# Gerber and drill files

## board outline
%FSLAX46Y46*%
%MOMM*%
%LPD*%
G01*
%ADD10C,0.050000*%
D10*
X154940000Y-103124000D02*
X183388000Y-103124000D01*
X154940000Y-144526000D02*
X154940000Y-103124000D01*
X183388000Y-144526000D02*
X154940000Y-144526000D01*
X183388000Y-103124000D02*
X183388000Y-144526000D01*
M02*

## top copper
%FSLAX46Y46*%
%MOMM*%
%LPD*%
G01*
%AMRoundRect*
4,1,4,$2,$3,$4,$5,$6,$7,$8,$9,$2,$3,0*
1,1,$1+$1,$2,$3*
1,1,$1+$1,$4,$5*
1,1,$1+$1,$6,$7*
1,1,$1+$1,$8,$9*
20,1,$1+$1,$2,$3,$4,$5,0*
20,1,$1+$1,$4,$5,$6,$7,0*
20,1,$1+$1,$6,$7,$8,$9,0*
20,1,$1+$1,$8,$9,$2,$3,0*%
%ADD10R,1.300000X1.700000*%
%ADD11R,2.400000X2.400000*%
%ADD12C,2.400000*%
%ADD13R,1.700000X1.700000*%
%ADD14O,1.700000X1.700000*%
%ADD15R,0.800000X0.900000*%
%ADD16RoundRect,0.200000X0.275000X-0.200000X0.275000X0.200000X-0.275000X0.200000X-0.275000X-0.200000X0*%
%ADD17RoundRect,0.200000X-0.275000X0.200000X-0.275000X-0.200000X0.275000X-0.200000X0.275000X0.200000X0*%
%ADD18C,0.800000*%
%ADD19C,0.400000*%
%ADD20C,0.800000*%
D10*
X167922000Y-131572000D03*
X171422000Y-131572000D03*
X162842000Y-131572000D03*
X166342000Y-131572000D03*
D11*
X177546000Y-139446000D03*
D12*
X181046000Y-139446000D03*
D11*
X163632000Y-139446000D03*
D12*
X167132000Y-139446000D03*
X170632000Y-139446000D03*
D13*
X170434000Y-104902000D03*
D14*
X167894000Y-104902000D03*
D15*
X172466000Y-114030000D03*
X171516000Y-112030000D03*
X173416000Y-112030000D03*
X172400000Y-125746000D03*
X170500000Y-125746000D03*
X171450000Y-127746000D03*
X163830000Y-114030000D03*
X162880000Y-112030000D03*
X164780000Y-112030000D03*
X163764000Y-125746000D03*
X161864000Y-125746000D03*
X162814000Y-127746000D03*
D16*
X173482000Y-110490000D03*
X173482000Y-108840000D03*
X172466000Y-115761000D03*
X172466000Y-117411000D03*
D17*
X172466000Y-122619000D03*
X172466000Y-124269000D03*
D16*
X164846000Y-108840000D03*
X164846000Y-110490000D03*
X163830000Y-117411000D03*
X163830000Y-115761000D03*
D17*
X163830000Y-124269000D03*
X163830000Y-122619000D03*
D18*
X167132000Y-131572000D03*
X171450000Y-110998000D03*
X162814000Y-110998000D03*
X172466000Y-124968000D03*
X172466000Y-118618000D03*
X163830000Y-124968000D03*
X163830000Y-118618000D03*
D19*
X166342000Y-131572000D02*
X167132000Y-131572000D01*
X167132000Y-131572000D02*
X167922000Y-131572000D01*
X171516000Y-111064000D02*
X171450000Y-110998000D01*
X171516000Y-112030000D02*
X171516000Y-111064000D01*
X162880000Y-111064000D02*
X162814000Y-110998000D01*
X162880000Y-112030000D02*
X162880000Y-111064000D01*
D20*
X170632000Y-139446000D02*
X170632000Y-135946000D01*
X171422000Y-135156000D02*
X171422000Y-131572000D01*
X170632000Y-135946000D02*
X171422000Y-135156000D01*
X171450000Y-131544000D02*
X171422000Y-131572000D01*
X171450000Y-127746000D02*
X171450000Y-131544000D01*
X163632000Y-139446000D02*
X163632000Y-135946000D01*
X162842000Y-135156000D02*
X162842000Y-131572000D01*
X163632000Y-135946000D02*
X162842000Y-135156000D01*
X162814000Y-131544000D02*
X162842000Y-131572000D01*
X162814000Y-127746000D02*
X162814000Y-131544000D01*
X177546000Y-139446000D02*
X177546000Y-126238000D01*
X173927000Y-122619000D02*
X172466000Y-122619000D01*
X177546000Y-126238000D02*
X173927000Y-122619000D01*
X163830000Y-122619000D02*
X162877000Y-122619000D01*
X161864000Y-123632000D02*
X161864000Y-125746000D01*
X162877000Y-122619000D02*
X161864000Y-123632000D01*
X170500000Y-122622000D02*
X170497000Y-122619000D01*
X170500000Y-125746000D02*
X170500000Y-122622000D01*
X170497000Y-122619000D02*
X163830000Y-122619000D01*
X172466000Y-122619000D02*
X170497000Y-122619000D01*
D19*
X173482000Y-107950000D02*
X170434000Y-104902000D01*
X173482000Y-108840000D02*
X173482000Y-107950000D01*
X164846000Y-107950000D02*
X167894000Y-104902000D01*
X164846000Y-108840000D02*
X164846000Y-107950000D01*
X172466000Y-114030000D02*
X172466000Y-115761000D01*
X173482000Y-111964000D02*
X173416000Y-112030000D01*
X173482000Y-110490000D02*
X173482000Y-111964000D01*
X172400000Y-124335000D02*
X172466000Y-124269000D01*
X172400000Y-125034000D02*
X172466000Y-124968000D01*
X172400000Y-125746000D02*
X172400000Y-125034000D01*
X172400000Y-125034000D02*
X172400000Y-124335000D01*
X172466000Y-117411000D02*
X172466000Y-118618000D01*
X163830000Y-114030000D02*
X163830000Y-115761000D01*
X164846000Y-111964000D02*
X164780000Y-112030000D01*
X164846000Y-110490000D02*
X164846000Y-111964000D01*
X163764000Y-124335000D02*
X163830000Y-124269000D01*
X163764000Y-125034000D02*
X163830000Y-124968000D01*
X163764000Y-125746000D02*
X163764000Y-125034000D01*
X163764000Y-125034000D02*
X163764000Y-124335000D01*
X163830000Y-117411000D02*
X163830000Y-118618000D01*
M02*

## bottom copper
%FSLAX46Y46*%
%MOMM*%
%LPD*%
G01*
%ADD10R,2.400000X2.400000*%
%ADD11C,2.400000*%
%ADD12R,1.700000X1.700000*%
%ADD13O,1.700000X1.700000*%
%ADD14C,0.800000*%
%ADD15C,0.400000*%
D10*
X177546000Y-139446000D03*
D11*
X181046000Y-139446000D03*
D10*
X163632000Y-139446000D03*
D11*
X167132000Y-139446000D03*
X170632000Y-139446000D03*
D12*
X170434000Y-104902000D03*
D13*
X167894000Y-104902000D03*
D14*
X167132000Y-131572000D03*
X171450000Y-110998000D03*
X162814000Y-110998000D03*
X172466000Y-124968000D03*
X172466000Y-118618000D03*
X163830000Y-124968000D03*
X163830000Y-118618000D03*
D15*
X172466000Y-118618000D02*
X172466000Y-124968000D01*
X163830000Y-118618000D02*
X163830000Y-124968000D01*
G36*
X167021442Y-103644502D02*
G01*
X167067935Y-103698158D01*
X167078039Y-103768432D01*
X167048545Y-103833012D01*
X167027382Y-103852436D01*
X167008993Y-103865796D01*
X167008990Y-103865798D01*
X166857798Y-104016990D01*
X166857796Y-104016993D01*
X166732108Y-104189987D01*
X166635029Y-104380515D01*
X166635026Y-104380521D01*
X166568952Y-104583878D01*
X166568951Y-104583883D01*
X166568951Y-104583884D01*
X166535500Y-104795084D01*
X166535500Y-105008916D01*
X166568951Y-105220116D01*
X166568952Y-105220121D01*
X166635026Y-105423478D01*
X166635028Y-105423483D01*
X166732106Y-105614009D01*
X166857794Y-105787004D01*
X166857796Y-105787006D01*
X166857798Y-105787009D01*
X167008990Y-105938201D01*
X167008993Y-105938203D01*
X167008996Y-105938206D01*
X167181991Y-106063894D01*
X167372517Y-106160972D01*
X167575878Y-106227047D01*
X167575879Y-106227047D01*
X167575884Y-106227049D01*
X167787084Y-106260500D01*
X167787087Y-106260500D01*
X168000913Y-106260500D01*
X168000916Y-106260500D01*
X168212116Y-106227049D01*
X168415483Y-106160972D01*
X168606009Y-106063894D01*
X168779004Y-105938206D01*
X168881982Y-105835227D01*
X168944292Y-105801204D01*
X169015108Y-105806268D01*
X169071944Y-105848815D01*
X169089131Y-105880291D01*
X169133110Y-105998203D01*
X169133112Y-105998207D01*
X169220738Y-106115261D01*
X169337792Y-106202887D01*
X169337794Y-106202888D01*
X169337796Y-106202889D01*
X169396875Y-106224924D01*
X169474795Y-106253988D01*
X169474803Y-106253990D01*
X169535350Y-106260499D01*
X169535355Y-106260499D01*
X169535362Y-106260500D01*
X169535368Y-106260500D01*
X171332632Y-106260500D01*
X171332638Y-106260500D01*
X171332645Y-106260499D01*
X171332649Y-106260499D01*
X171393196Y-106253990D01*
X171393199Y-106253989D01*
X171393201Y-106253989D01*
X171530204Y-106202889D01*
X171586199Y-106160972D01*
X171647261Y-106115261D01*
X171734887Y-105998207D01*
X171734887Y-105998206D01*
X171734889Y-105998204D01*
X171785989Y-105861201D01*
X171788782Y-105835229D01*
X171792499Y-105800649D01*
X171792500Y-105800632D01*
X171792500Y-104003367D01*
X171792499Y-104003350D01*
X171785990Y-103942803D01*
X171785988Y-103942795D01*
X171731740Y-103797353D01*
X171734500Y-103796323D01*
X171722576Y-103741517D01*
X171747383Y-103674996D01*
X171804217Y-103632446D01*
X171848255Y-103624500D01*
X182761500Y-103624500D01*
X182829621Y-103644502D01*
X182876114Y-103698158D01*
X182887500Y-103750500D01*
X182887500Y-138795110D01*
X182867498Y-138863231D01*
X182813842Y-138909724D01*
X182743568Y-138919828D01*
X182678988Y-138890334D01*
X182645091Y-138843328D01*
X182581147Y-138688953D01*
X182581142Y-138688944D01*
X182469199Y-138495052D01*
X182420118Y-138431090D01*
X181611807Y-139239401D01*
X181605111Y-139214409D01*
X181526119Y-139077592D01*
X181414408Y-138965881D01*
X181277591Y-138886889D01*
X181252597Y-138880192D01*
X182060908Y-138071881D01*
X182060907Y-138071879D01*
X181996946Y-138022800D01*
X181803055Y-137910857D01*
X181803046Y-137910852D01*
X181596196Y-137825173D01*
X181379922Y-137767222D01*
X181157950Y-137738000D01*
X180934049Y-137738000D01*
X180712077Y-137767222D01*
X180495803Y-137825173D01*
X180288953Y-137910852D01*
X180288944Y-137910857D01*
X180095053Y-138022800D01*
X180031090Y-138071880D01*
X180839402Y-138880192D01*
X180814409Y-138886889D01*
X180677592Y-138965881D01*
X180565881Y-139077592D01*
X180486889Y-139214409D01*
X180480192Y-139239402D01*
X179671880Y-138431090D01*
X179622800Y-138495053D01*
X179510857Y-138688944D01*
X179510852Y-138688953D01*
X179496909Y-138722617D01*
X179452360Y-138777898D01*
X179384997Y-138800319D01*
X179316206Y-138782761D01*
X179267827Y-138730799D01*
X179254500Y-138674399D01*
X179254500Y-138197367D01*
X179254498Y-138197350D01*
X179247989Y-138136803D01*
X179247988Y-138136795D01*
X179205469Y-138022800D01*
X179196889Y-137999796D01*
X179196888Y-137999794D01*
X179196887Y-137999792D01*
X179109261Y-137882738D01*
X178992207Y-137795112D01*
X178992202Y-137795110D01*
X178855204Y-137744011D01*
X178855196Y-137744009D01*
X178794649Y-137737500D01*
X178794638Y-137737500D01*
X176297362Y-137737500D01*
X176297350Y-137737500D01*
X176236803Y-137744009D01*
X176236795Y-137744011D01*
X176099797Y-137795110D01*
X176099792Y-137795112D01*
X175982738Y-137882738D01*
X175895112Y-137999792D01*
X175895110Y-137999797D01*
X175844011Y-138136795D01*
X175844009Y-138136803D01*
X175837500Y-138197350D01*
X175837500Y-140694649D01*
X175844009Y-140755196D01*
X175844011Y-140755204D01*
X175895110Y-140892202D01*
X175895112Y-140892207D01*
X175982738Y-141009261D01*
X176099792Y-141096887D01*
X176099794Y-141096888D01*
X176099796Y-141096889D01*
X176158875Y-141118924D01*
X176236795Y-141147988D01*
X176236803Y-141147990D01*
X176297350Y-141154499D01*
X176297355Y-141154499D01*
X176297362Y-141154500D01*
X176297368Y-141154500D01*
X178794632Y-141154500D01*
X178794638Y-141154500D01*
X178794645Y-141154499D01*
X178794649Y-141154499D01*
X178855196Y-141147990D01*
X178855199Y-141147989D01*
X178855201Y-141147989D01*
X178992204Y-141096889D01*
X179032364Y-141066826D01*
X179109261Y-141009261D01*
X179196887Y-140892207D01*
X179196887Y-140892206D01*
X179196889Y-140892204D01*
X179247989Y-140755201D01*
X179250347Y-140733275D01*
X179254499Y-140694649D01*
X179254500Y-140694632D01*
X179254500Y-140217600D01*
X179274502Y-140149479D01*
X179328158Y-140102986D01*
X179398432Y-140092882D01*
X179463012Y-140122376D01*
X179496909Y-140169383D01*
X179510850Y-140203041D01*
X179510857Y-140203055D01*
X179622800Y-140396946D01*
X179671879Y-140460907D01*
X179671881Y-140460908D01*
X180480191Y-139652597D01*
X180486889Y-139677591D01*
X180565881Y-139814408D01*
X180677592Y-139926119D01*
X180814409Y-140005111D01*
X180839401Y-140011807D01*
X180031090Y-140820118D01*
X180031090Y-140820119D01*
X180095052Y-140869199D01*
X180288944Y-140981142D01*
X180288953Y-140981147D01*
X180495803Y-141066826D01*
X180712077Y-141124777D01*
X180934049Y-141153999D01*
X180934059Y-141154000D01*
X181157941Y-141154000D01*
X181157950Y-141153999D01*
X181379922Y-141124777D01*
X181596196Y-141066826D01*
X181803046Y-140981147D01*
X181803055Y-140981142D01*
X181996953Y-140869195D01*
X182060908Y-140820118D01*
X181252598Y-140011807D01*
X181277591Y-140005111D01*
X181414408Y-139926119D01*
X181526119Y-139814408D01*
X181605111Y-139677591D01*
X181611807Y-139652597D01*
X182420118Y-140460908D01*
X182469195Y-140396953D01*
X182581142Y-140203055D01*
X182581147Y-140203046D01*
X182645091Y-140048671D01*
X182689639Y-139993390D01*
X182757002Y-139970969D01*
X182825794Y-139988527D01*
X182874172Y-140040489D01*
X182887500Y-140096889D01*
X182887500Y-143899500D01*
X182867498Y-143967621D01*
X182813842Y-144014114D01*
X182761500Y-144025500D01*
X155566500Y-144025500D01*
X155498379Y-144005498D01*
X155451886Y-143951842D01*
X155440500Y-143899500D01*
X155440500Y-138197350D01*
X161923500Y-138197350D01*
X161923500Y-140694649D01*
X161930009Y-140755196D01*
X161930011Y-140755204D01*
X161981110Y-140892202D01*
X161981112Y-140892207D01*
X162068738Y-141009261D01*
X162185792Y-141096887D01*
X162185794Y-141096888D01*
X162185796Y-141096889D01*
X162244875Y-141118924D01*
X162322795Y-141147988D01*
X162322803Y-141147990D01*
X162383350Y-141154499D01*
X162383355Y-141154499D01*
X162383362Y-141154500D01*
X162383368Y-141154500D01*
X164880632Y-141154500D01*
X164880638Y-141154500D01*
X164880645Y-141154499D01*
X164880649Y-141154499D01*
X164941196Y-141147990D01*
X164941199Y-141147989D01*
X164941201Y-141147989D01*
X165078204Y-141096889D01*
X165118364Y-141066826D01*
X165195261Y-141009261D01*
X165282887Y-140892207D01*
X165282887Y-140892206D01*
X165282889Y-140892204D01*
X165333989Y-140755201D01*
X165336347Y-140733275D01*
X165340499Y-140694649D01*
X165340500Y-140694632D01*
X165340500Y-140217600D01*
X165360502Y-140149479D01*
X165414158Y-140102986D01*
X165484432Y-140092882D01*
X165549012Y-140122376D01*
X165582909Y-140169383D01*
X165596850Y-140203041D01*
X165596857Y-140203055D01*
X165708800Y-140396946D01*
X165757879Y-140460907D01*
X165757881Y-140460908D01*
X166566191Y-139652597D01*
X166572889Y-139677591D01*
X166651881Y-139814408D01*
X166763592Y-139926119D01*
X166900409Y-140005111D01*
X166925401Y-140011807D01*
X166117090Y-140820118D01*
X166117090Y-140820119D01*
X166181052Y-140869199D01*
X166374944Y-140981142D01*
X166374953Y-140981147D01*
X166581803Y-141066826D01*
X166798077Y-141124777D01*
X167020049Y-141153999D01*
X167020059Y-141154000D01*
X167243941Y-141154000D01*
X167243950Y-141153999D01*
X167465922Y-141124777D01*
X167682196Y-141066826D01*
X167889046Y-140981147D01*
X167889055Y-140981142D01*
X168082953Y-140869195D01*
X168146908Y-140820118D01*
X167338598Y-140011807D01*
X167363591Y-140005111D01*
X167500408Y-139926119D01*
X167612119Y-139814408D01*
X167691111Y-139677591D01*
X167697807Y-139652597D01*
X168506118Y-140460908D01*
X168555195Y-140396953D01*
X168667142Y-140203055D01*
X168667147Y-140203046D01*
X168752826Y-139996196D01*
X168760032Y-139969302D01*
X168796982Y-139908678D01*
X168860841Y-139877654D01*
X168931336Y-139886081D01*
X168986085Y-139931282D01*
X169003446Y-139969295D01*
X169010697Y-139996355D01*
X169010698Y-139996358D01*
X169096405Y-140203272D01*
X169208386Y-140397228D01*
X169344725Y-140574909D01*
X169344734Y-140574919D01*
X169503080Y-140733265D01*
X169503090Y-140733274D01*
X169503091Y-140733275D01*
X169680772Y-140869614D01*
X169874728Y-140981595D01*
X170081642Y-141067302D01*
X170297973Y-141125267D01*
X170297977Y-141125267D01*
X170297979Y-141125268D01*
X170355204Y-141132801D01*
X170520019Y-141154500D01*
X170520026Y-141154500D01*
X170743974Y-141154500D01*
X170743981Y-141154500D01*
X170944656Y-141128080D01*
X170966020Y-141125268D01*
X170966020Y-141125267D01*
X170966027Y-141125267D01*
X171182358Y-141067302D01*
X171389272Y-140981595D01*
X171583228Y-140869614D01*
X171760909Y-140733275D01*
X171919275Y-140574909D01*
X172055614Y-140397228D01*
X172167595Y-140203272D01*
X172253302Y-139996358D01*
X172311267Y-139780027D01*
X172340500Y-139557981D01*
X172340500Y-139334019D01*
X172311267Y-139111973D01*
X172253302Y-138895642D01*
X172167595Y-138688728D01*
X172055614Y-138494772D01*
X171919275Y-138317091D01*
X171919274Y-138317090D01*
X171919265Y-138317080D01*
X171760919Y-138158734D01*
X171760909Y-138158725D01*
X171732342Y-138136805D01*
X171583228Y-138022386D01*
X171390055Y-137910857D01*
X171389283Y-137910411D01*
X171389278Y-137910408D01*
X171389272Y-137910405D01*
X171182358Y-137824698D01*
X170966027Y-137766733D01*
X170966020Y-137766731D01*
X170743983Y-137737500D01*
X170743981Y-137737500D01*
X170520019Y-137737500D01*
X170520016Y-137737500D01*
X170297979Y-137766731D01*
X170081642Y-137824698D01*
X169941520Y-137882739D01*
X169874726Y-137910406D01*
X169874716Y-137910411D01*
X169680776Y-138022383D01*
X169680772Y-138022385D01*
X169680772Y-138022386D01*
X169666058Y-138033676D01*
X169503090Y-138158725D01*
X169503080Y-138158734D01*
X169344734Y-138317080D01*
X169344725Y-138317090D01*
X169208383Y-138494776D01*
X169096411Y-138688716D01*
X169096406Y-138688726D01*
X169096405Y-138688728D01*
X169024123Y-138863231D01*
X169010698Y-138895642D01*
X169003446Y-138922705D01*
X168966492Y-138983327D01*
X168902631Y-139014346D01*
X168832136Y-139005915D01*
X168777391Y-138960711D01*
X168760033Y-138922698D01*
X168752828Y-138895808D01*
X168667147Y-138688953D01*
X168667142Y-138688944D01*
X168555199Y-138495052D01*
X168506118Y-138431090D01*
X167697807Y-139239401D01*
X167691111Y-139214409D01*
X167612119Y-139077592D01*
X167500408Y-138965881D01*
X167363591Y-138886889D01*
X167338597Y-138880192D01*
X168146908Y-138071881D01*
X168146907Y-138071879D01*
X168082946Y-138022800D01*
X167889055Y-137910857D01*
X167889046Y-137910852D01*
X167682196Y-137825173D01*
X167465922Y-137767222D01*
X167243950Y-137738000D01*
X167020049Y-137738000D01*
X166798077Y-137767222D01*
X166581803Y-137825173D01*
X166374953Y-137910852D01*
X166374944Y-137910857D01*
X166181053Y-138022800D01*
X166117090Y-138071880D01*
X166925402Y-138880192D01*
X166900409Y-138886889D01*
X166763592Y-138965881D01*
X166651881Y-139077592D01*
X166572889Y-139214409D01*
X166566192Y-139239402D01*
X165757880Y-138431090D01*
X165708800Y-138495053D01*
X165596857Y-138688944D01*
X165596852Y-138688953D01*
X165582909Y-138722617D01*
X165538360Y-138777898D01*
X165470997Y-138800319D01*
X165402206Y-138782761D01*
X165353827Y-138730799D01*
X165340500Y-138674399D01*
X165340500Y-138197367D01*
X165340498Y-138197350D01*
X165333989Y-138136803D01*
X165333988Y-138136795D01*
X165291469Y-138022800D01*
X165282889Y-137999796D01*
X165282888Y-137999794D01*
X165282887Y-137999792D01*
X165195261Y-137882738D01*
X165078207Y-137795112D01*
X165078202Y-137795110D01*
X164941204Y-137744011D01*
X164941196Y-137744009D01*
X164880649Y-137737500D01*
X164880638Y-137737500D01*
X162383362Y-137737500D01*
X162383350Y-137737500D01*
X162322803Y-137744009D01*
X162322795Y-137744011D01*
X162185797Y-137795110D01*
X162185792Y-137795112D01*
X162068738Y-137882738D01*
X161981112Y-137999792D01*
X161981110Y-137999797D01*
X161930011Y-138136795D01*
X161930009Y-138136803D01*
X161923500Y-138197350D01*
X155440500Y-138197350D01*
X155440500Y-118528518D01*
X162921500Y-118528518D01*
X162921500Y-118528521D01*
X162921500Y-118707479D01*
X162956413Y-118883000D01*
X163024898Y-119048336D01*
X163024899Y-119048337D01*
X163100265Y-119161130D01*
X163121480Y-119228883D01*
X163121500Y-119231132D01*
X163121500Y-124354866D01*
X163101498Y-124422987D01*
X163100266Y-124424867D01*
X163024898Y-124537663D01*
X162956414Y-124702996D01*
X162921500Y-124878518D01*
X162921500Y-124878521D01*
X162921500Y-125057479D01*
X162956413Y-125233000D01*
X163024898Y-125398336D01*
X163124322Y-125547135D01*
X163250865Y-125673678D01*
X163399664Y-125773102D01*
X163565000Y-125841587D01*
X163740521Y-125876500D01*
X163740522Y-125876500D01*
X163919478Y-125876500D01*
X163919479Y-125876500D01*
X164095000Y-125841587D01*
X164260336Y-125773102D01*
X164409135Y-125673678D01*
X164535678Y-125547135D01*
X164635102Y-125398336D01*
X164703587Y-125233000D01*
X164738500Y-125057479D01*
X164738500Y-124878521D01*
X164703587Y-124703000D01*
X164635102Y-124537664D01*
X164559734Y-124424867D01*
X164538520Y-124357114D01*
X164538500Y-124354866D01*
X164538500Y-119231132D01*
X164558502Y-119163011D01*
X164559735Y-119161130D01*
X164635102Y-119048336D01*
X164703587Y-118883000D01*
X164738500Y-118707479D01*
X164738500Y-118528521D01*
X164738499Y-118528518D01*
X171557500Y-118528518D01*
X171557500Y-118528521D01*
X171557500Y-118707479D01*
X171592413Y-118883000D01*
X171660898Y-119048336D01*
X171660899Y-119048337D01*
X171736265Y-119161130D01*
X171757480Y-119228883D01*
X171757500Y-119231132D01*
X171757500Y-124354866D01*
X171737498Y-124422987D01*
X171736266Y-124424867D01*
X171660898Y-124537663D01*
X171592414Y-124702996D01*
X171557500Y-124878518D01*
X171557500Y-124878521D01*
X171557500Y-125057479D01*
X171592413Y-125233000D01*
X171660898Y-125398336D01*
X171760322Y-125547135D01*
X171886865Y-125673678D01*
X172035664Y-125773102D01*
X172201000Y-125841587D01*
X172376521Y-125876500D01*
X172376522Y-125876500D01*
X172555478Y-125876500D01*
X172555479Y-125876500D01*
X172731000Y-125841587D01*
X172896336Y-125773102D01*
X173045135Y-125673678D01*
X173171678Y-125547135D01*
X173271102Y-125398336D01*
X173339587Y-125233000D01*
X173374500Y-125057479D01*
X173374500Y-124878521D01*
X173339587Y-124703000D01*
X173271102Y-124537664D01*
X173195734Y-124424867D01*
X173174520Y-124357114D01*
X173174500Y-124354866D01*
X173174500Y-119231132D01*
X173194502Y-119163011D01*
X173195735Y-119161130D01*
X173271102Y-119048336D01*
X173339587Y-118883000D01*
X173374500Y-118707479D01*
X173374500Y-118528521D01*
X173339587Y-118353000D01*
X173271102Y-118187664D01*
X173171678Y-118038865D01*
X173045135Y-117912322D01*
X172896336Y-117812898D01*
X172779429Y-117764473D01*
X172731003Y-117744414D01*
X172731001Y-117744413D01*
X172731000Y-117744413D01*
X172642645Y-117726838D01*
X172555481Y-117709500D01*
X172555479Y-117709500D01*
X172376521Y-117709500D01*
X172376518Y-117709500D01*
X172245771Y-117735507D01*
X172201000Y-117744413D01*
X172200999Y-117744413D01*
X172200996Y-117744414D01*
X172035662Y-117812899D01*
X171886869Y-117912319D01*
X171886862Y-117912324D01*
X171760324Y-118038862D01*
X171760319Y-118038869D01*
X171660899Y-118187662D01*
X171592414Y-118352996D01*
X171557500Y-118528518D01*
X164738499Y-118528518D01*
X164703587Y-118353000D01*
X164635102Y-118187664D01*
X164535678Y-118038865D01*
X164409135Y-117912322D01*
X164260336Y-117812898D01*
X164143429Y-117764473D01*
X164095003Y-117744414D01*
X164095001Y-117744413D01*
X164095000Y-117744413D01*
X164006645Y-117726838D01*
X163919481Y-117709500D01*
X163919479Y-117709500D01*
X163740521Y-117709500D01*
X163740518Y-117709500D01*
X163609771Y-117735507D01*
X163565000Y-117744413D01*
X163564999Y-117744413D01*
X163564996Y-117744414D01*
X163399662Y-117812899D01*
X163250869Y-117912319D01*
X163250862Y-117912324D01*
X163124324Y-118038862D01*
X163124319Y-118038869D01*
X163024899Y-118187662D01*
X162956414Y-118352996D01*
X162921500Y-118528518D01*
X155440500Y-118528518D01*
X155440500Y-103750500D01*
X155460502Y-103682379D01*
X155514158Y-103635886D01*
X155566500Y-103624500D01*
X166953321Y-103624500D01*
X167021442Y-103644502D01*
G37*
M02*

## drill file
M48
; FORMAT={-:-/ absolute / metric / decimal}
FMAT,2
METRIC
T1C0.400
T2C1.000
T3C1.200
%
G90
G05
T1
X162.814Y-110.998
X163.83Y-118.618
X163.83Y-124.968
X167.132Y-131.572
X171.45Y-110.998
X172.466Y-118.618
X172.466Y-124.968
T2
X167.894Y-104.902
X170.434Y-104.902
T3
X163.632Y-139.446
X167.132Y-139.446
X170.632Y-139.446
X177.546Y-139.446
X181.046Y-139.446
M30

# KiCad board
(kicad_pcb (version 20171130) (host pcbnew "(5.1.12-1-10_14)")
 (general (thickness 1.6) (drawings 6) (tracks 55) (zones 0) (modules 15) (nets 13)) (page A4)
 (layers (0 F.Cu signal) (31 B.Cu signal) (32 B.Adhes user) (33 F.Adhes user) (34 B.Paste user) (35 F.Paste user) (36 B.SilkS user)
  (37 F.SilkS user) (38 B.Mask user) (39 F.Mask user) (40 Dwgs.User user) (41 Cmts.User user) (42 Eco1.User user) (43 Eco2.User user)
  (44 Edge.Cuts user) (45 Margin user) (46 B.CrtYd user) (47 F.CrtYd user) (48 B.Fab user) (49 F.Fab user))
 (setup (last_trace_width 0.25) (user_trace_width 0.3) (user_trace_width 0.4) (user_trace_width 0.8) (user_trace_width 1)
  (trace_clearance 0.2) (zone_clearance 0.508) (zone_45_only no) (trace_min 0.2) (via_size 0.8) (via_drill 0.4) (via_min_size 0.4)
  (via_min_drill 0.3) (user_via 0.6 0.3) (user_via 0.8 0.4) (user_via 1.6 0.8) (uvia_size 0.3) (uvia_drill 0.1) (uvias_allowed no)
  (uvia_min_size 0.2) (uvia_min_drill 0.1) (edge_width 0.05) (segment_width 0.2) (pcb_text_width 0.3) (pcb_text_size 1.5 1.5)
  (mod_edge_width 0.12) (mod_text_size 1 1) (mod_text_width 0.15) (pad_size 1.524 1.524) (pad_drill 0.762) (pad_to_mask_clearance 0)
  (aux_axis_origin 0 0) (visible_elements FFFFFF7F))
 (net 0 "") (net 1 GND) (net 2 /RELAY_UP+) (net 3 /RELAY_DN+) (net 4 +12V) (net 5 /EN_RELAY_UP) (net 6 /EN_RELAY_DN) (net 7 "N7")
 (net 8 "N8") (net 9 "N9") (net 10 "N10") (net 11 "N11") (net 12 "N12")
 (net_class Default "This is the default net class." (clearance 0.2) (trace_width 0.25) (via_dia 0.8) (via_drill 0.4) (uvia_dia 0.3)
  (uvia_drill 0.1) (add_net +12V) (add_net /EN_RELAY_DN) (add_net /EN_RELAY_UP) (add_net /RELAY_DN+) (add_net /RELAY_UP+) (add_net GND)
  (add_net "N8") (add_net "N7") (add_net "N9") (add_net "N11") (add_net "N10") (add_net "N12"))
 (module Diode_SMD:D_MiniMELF (layer F.Cu) (at 169.672 131.572 180)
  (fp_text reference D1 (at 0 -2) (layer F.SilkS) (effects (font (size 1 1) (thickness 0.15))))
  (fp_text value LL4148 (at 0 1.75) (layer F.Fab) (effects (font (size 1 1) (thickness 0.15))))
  (pad 2 smd rect (at 1.75 0 180) (size 1.3 1.7) (layers F.Cu F.Paste F.Mask) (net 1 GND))
  (pad 1 smd rect (at -1.75 0 180) (size 1.3 1.7) (layers F.Cu F.Paste F.Mask) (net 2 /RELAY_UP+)))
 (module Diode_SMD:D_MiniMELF (layer F.Cu) (at 164.592 131.572)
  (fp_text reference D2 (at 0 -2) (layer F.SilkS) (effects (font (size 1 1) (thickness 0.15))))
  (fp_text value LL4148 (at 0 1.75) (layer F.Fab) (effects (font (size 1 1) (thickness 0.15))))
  (pad 1 smd rect (at -1.75 0) (size 1.3 1.7) (layers F.Cu F.Paste F.Mask) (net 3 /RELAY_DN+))
  (pad 2 smd rect (at 1.75 0) (size 1.3 1.7) (layers F.Cu F.Paste F.Mask) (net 1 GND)))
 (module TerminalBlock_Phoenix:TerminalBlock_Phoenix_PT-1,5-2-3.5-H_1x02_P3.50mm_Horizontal (layer F.Cu) (at 177.546 139.446)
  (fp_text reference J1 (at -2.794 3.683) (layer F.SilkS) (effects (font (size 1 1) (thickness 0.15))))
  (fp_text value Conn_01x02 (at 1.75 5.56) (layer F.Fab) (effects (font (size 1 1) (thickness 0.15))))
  (pad 1 thru_hole rect (at 0 0) (size 2.4 2.4) (drill 1.2) (layers *.Cu *.Mask) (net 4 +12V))
  (pad 2 thru_hole circle (at 3.5 0) (size 2.4 2.4) (drill 1.2) (layers *.Cu *.Mask) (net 1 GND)))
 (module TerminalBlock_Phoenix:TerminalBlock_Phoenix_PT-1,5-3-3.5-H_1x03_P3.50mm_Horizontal (layer F.Cu) (at 163.632 139.446)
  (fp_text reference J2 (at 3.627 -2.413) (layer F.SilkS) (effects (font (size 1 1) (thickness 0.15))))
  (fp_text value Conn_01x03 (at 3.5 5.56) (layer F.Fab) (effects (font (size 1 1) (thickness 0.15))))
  (pad 1 thru_hole rect (at 0 0) (size 2.4 2.4) (drill 1.2) (layers *.Cu *.Mask) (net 3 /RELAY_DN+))
  (pad 2 thru_hole circle (at 3.5 0) (size 2.4 2.4) (drill 1.2) (layers *.Cu *.Mask) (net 1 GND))
  (pad 3 thru_hole circle (at 7 0) (size 2.4 2.4) (drill 1.2) (layers *.Cu *.Mask) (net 2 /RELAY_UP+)))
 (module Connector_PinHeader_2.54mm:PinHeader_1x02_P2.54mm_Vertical (layer F.Cu) (at 170.434 104.902 270)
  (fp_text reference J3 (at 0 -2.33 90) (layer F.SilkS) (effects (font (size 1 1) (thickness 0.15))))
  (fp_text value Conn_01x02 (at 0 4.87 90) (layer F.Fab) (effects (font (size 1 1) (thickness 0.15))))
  (pad 1 thru_hole rect (at 0 0 270) (size 1.7 1.7) (drill 1) (layers *.Cu *.Mask) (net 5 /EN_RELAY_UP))
  (pad 2 thru_hole oval (at 0 2.54 270) (size 1.7 1.7) (drill 1) (layers *.Cu *.Mask) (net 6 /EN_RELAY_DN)))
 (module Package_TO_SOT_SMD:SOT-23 (layer F.Cu) (at 172.466 113.03 270)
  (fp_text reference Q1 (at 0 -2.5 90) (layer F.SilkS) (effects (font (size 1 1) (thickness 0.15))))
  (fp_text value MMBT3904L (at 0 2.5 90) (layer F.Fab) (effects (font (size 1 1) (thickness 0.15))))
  (pad 3 smd rect (at 1 0 270) (size 0.9 0.8) (layers F.Cu F.Paste F.Mask) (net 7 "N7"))
  (pad 2 smd rect (at -1 0.95 270) (size 0.9 0.8) (layers F.Cu F.Paste F.Mask) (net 1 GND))
  (pad 1 smd rect (at -1 -0.95 270) (size 0.9 0.8) (layers F.Cu F.Paste F.Mask) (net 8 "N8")))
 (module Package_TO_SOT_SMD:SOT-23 (layer F.Cu) (at 171.45 126.746 270)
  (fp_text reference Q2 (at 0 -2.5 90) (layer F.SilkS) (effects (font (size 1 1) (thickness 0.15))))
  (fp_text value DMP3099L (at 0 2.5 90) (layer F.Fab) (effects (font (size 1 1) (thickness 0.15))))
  (pad 1 smd rect (at -1 -0.95 270) (size 0.9 0.8) (layers F.Cu F.Paste F.Mask) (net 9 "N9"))
  (pad 2 smd rect (at -1 0.95 270) (size 0.9 0.8) (layers F.Cu F.Paste F.Mask) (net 4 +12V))
  (pad 3 smd rect (at 1 0 270) (size 0.9 0.8) (layers F.Cu F.Paste F.Mask) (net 2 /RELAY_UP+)))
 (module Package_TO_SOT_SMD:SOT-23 (layer F.Cu) (at 163.83 113.03 270)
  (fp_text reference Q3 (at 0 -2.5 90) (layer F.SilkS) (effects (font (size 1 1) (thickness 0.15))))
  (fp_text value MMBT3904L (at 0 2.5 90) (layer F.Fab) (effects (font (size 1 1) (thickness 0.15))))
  (pad 3 smd rect (at 1 0 270) (size 0.9 0.8) (layers F.Cu F.Paste F.Mask) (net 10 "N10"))
  (pad 2 smd rect (at -1 0.95 270) (size 0.9 0.8) (layers F.Cu F.Paste F.Mask) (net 1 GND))
  (pad 1 smd rect (at -1 -0.95 270) (size 0.9 0.8) (layers F.Cu F.Paste F.Mask) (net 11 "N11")))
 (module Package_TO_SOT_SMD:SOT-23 (layer F.Cu) (at 162.814 126.746 270)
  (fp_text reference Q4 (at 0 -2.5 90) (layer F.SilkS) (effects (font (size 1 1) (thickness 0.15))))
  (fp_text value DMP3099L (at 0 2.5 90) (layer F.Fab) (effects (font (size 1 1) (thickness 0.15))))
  (pad 1 smd rect (at -1 -0.95 270) (size 0.9 0.8) (layers F.Cu F.Paste F.Mask) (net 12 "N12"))
  (pad 2 smd rect (at -1 0.95 270) (size 0.9 0.8) (layers F.Cu F.Paste F.Mask) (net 4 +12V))
  (pad 3 smd rect (at 1 0 270) (size 0.9 0.8) (layers F.Cu F.Paste F.Mask) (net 3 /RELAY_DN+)))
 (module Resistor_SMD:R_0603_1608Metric (layer F.Cu) (at 173.482 109.665 90)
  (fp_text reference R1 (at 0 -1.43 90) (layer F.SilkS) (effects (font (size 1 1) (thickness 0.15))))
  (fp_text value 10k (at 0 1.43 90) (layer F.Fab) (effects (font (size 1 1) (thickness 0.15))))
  (pad 1 smd roundrect (at -0.825 0 90) (size 0.8 0.95) (layers F.Cu F.Paste F.Mask) (roundrect_rratio 0.25) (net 8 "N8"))
  (pad 2 smd roundrect (at 0.825 0 90) (size 0.8 0.95) (layers F.Cu F.Paste F.Mask) (roundrect_rratio 0.25) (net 5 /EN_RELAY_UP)))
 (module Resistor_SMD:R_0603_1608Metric (layer F.Cu) (at 172.466 116.586 90)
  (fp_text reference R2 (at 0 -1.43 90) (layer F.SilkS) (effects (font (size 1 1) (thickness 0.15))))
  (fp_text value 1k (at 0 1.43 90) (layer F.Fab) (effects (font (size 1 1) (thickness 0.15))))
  (pad 2 smd roundrect (at 0.825 0 90) (size 0.8 0.95) (layers F.Cu F.Paste F.Mask) (roundrect_rratio 0.25) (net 7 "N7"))
  (pad 1 smd roundrect (at -0.825 0 90) (size 0.8 0.95) (layers F.Cu F.Paste F.Mask) (roundrect_rratio 0.25) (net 9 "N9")))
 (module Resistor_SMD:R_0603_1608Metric (layer F.Cu) (at 172.466 123.444 270)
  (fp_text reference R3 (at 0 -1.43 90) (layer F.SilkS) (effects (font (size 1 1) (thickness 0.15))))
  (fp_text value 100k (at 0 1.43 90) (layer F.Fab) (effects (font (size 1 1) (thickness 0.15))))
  (pad 1 smd roundrect (at -0.825 0 270) (size 0.8 0.95) (layers F.Cu F.Paste F.Mask) (roundrect_rratio 0.25) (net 4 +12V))
  (pad 2 smd roundrect (at 0.825 0 270) (size 0.8 0.95) (layers F.Cu F.Paste F.Mask) (roundrect_rratio 0.25) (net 9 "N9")))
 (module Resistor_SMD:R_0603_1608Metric (layer F.Cu) (at 164.846 109.665 90)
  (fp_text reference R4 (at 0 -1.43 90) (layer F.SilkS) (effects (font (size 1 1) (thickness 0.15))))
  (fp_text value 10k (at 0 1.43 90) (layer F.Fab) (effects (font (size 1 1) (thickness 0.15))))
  (pad 2 smd roundrect (at 0.825 0 90) (size 0.8 0.95) (layers F.Cu F.Paste F.Mask) (roundrect_rratio 0.25) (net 6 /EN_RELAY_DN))
  (pad 1 smd roundrect (at -0.825 0 90) (size 0.8 0.95) (layers F.Cu F.Paste F.Mask) (roundrect_rratio 0.25) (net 11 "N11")))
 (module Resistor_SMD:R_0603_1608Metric (layer F.Cu) (at 163.83 116.586 90)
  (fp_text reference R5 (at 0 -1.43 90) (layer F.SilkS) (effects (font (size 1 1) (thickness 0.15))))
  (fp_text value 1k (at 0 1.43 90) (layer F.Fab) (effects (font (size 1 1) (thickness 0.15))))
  (pad 1 smd roundrect (at -0.825 0 90) (size 0.8 0.95) (layers F.Cu F.Paste F.Mask) (roundrect_rratio 0.25) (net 12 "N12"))
  (pad 2 smd roundrect (at 0.825 0 90) (size 0.8 0.95) (layers F.Cu F.Paste F.Mask) (roundrect_rratio 0.25) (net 10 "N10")))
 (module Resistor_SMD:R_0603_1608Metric (layer F.Cu) (at 163.83 123.444 270)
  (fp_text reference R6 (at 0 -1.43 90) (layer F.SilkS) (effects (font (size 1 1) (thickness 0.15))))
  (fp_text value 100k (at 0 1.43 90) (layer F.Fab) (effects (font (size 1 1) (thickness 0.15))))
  (pad 2 smd roundrect (at 0.825 0 270) (size 0.8 0.95) (layers F.Cu F.Paste F.Mask) (roundrect_rratio 0.25) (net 12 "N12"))
  (pad 1 smd roundrect (at -0.825 0 270) (size 0.8 0.95) (layers F.Cu F.Paste F.Mask) (roundrect_rratio 0.25) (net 4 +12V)))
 (gr_line (start 154.94 103.124) (end 183.388 103.124) (layer Edge.Cuts) (width 0.05))
 (gr_line (start 154.94 144.526) (end 154.94 103.124) (layer Edge.Cuts) (width 0.05))
 (gr_line (start 183.388 144.526) (end 154.94 144.526) (layer Edge.Cuts) (width 0.05))
 (gr_line (start 183.388 103.124) (end 183.388 144.526) (layer Edge.Cuts) (width 0.05))
 (segment (start 166.342 131.572) (end 167.132 131.572) (width 0.4) (layer F.Cu) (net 1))
 (via (at 167.132 131.572) (size 0.8) (drill 0.4) (layers F.Cu B.Cu) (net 1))
 (segment (start 167.132 131.572) (end 167.922 131.572) (width 0.4) (layer F.Cu) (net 1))
 (via (at 171.45 110.998) (size 0.8) (drill 0.4) (layers F.Cu B.Cu) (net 1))
 (segment (start 171.516 111.064) (end 171.45 110.998) (width 0.4) (layer F.Cu) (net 1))
 (segment (start 171.516 112.03) (end 171.516 111.064) (width 0.4) (layer F.Cu) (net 1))
 (via (at 162.814 110.998) (size 0.8) (drill 0.4) (layers F.Cu B.Cu) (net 1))
 (segment (start 162.88 111.064) (end 162.814 110.998) (width 0.4) (layer F.Cu) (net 1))
 (segment (start 162.88 112.03) (end 162.88 111.064) (width 0.4) (layer F.Cu) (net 1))
 (segment (start 170.632 139.446) (end 170.632 135.946) (width 0.8) (layer F.Cu) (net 2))
 (segment (start 171.422 135.156) (end 171.422 131.572) (width 0.8) (layer F.Cu) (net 2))
 (segment (start 170.632 135.946) (end 171.422 135.156) (width 0.8) (layer F.Cu) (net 2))
 (segment (start 171.45 131.544) (end 171.422 131.572) (width 0.8) (layer F.Cu) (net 2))
 (segment (start 171.45 127.746) (end 171.45 131.544) (width 0.8) (layer F.Cu) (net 2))
 (segment (start 163.632 139.446) (end 163.632 135.946) (width 0.8) (layer F.Cu) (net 3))
 (segment (start 162.842 135.156) (end 162.842 131.572) (width 0.8) (layer F.Cu) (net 3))
 (segment (start 163.632 135.946) (end 162.842 135.156) (width 0.8) (layer F.Cu) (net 3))
 (segment (start 162.814 131.544) (end 162.842 131.572) (width 0.8) (layer F.Cu) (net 3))
 (segment (start 162.814 127.746) (end 162.814 131.544) (width 0.8) (layer F.Cu) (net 3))
 (segment (start 177.546 139.446) (end 177.546 126.238) (width 0.8) (layer F.Cu) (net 4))
 (segment (start 173.927 122.619) (end 172.466 122.619) (width 0.8) (layer F.Cu) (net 4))
 (segment (start 177.546 126.238) (end 173.927 122.619) (width 0.8) (layer F.Cu) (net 4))
 (segment (start 163.83 122.619) (end 162.877 122.619) (width 0.8) (layer F.Cu) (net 4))
 (segment (start 161.864 123.632) (end 161.864 125.746) (width 0.8) (layer F.Cu) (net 4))
 (segment (start 162.877 122.619) (end 161.864 123.632) (width 0.8) (layer F.Cu) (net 4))
 (segment (start 170.5 122.622) (end 170.497 122.619) (width 0.8) (layer F.Cu) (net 4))
 (segment (start 170.5 125.746) (end 170.5 122.622) (width 0.8) (layer F.Cu) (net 4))
 (segment (start 170.497 122.619) (end 163.83 122.619) (width 0.8) (layer F.Cu) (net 4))
 (segment (start 172.466 122.619) (end 170.497 122.619) (width 0.8) (layer F.Cu) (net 4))
 (segment (start 173.482 107.95) (end 170.434 104.902) (width 0.4) (layer F.Cu) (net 5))
 (segment (start 173.482 108.84) (end 173.482 107.95) (width 0.4) (layer F.Cu) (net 5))
 (segment (start 164.846 107.95) (end 167.894 104.902) (width 0.4) (layer F.Cu) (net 6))
 (segment (start 164.846 108.84) (end 164.846 107.95) (width 0.4) (layer F.Cu) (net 6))
 (segment (start 172.466 114.03) (end 172.466 115.761) (width 0.4) (layer F.Cu) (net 7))
 (segment (start 173.482 111.964) (end 173.416 112.03) (width 0.4) (layer F.Cu) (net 8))
 (segment (start 173.482 110.49) (end 173.482 111.964) (width 0.4) (layer F.Cu) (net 8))
 (segment (start 172.4 124.335) (end 172.466 124.269) (width 0.4) (layer F.Cu) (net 9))
 (segment (start 172.4 125.034) (end 172.466 124.968) (width 0.4) (layer F.Cu) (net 9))
 (segment (start 172.4 125.746) (end 172.4 125.034) (width 0.4) (layer F.Cu) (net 9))
 (via (at 172.466 124.968) (size 0.8) (drill 0.4) (layers F.Cu B.Cu) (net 9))
 (segment (start 172.4 125.034) (end 172.4 124.335) (width 0.4) (layer F.Cu) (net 9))
 (via (at 172.466 118.618) (size 0.8) (drill 0.4) (layers F.Cu B.Cu) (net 9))
 (segment (start 172.466 117.411) (end 172.466 118.618) (width 0.4) (layer F.Cu) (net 9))
 (segment (start 172.466 118.618) (end 172.466 124.968) (width 0.4) (layer B.Cu) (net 9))
 (segment (start 163.83 114.03) (end 163.83 115.761) (width 0.4) (layer F.Cu) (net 10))
 (segment (start 164.846 111.964) (end 164.78 112.03) (width 0.4) (layer F.Cu) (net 11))
 (segment (start 164.846 110.49) (end 164.846 111.964) (width 0.4) (layer F.Cu) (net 11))
 (segment (start 163.764 124.335) (end 163.83 124.269) (width 0.4) (layer F.Cu) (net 12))
 (via (at 163.83 124.968) (size 0.8) (drill 0.4) (layers F.Cu B.Cu) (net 12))
 (segment (start 163.764 125.034) (end 163.83 124.968) (width 0.4) (layer F.Cu) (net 12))
 (segment (start 163.764 125.746) (end 163.764 125.034) (width 0.4) (layer F.Cu) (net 12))
 (segment (start 163.764 125.034) (end 163.764 124.335) (width 0.4) (layer F.Cu) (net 12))
 (via (at 163.83 118.618) (size 0.8) (drill 0.4) (layers F.Cu B.Cu) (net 12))
 (segment (start 163.83 117.411) (end 163.83 118.618) (width 0.4) (layer F.Cu) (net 12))
 (segment (start 163.83 118.618) (end 163.83 124.968) (width 0.4) (layer B.Cu) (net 12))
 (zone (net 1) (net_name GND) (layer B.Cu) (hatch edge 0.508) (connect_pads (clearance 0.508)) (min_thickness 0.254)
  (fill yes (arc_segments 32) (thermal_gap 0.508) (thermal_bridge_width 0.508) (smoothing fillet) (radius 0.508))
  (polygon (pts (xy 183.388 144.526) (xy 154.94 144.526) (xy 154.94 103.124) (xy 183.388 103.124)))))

